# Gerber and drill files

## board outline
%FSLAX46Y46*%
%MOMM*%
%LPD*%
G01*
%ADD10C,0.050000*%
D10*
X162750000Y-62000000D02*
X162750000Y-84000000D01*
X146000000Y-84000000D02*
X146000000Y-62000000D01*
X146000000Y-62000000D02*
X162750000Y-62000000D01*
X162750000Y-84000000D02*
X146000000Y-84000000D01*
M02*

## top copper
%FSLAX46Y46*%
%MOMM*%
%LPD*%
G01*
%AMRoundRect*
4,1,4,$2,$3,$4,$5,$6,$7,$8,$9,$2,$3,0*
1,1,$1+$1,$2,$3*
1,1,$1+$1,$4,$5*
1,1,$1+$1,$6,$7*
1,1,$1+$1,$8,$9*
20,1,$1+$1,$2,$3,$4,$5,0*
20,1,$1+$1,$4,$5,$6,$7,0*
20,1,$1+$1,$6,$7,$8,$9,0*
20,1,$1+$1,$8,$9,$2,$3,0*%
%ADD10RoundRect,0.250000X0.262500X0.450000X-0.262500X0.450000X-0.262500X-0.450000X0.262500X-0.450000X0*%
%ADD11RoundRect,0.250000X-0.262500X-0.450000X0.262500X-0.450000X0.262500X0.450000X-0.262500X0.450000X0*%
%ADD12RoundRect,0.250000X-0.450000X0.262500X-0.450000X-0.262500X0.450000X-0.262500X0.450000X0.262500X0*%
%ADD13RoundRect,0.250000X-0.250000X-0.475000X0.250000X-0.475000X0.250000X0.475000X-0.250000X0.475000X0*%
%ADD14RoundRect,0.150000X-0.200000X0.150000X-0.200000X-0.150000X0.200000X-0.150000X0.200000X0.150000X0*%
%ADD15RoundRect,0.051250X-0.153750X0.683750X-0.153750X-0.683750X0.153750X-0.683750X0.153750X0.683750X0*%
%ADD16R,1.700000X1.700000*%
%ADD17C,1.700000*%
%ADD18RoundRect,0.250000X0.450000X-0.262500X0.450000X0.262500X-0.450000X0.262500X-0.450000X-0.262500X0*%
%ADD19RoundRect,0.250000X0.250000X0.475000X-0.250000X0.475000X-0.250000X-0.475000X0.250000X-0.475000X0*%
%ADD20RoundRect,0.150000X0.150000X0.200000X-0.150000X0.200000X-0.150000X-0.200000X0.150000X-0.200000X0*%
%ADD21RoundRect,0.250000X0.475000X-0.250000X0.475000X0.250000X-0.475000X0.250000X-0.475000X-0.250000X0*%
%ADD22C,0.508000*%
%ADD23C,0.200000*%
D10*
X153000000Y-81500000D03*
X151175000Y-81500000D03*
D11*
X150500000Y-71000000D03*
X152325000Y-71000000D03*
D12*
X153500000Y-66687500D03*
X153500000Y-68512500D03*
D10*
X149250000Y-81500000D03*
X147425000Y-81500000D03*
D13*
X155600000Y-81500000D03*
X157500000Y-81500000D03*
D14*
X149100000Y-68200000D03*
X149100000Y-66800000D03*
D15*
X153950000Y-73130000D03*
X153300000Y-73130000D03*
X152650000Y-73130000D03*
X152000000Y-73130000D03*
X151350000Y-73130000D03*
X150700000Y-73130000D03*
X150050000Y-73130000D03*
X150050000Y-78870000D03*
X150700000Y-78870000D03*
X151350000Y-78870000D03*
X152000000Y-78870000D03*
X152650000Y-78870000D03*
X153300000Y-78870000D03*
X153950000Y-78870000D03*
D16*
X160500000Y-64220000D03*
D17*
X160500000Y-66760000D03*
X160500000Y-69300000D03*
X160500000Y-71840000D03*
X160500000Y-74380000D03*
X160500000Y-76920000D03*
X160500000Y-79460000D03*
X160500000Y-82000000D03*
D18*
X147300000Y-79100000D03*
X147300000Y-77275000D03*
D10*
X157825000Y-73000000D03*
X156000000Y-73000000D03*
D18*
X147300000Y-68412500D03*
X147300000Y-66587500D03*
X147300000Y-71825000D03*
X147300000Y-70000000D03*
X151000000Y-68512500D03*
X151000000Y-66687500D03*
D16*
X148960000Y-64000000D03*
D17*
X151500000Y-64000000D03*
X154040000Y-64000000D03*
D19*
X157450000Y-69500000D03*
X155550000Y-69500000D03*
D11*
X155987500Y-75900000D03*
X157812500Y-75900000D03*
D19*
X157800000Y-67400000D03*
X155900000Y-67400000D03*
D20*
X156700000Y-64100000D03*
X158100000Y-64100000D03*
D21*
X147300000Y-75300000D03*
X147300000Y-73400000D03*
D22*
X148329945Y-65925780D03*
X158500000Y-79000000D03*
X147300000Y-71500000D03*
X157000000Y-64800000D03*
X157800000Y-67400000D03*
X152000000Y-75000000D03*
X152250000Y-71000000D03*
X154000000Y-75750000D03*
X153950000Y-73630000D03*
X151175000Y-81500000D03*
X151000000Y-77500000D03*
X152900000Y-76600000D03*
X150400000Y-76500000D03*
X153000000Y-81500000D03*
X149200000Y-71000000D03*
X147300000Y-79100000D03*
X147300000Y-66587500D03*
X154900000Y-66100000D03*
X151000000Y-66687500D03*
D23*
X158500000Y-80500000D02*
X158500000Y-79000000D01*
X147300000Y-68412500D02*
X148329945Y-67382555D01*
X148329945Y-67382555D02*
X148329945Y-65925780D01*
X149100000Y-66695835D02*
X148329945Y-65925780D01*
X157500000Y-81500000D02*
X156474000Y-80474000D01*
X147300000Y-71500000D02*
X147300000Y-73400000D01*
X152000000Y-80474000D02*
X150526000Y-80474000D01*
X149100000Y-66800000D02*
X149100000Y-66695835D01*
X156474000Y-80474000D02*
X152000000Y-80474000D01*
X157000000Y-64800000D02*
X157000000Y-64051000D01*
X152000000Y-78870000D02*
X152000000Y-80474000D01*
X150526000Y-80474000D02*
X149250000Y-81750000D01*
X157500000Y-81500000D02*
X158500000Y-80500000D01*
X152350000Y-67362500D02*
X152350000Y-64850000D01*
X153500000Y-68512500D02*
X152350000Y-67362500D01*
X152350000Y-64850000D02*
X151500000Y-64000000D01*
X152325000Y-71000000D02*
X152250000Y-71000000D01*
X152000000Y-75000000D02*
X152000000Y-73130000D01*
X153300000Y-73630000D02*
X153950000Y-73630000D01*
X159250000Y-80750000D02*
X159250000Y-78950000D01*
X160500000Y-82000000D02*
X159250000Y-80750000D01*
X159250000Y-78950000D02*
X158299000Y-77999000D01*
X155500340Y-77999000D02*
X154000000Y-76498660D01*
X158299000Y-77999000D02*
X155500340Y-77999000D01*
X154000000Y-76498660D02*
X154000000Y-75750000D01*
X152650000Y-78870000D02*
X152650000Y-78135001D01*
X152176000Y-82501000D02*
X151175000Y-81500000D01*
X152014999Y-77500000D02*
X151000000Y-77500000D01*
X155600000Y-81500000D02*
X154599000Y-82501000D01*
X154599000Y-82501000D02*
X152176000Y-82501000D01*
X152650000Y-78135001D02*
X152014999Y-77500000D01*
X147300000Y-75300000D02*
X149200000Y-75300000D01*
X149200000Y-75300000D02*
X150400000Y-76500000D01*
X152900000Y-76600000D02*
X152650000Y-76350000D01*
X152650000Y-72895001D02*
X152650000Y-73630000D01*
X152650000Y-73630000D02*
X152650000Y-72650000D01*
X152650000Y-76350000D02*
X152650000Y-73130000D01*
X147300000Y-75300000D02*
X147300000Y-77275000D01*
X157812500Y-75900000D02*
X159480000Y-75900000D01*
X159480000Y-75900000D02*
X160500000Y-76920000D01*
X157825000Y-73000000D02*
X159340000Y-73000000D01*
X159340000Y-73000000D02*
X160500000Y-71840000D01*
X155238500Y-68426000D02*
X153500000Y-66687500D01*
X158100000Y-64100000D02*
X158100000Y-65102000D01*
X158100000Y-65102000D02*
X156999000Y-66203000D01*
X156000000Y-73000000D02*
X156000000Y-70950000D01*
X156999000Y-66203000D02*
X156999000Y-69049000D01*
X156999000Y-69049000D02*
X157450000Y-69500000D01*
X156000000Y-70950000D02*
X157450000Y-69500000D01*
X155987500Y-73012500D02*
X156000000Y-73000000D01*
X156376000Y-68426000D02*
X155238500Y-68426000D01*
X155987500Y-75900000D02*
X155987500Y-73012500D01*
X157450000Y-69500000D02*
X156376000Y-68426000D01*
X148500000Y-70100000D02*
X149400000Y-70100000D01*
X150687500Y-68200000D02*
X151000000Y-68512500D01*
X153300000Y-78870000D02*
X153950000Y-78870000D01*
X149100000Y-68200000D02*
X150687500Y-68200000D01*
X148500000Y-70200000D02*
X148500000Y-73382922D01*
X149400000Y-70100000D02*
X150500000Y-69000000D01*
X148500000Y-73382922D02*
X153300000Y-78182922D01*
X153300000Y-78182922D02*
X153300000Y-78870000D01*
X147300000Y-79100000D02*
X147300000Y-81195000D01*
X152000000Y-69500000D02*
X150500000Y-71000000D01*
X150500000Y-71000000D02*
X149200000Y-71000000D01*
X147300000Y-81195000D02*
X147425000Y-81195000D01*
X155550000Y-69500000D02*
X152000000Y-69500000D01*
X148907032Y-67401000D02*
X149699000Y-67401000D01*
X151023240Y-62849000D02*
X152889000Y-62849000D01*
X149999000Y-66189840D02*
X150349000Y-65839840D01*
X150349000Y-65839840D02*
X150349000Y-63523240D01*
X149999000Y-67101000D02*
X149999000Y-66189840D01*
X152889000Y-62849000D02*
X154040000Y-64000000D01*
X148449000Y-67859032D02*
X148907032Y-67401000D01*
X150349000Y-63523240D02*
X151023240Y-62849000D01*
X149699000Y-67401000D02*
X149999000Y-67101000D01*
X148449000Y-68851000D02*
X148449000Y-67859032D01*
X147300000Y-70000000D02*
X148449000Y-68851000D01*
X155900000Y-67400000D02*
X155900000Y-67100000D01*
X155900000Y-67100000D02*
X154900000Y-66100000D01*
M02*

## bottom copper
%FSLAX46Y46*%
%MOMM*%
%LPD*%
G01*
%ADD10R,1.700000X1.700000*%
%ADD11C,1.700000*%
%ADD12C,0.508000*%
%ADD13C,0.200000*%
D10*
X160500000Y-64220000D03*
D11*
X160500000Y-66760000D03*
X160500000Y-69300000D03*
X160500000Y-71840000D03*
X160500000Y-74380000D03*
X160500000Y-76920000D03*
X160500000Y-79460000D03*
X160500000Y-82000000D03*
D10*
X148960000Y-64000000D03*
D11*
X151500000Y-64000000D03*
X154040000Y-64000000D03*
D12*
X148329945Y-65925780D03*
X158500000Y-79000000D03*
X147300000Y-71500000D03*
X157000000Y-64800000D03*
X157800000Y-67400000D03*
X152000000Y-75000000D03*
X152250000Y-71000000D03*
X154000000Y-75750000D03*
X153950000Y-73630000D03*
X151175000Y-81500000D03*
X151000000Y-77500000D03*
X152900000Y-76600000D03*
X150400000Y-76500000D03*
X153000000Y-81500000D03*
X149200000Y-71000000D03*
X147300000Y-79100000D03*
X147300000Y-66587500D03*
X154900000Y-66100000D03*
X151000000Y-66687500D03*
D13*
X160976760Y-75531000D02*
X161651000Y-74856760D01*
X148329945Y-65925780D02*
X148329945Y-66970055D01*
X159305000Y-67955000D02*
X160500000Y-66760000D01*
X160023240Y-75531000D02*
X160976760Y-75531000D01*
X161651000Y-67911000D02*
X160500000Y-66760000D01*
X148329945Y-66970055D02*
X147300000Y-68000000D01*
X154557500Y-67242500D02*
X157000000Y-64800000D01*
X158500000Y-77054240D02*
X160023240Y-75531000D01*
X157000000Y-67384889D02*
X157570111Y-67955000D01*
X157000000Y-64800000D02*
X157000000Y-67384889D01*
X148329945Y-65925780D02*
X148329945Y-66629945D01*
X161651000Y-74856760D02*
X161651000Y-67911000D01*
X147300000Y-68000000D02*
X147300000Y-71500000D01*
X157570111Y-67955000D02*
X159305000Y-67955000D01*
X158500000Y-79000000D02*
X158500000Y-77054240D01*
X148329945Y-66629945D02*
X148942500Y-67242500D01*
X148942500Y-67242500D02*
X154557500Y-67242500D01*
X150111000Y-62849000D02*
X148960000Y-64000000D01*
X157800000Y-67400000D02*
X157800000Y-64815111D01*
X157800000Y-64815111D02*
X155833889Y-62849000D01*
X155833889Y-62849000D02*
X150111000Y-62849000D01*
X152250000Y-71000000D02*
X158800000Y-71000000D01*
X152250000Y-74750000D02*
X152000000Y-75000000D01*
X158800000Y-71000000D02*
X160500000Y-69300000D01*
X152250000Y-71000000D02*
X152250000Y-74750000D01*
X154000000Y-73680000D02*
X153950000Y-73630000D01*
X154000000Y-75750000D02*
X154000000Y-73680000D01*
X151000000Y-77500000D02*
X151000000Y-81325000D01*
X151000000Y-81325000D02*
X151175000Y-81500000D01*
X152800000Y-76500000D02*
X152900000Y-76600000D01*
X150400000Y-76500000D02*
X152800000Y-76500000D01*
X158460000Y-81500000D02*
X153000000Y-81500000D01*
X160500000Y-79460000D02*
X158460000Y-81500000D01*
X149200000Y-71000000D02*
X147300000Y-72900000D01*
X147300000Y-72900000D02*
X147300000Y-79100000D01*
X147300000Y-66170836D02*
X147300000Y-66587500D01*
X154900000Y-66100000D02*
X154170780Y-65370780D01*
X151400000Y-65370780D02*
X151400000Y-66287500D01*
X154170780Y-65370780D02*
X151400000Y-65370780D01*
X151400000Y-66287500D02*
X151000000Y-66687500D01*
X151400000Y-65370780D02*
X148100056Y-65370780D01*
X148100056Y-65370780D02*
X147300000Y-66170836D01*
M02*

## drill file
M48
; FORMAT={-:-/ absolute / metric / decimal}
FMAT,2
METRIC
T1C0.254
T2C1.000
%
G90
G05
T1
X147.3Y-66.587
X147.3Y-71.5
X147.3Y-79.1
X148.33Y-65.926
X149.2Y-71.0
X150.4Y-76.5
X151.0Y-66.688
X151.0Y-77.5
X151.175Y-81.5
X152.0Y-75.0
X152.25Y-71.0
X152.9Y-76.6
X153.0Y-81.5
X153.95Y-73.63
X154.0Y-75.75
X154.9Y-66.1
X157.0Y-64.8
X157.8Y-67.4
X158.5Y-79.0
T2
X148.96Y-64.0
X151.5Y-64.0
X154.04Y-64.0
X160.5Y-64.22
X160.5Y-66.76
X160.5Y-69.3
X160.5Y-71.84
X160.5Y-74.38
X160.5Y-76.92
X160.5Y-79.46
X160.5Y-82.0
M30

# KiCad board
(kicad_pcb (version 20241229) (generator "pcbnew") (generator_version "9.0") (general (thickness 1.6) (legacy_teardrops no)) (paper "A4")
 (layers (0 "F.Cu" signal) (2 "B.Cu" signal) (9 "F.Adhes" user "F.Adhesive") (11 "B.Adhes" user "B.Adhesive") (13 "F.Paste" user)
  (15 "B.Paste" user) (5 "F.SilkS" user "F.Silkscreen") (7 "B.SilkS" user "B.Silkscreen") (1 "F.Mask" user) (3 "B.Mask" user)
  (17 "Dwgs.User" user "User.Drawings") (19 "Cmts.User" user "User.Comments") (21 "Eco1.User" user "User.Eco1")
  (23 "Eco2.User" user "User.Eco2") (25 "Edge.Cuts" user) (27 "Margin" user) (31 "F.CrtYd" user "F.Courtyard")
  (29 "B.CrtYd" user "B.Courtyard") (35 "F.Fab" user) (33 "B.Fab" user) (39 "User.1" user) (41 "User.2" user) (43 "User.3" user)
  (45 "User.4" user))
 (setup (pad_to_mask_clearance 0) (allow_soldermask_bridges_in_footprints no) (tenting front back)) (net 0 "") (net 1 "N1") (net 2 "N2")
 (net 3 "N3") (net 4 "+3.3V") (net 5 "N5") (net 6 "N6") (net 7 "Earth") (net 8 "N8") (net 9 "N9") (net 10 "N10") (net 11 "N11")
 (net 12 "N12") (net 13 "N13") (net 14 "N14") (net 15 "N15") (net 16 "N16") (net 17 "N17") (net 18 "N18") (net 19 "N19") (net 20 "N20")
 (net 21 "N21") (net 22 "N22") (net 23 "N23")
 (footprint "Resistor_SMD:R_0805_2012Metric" (layer "F.Cu") (at 152.0875 81.5 180)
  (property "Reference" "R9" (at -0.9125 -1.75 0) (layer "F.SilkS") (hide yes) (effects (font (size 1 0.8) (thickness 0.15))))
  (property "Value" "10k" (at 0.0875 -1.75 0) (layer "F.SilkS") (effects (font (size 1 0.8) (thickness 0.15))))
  (pad "1" smd roundrect (at -0.9125 0 180) (size 1.025 1.4) (layers "F.Cu" "F.Mask" "F.Paste") (roundrect_rratio 0.243902) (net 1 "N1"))
  (pad "2" smd roundrect (at 0.9125 0 180) (size 1.025 1.4) (layers "F.Cu" "F.Mask" "F.Paste") (roundrect_rratio 0.243902) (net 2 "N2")))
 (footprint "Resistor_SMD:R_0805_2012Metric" (layer "F.Cu") (at 151.4125 71)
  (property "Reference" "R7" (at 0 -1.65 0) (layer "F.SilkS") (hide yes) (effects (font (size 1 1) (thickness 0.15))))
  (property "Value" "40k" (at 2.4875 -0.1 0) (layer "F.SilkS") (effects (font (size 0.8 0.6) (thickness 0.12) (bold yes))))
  (pad "1" smd roundrect (at -0.9125 0) (size 1.025 1.4) (layers "F.Cu" "F.Mask" "F.Paste") (roundrect_rratio 0.243902) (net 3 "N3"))
  (pad "2" smd roundrect (at 0.9125 0) (size 1.025 1.4) (layers "F.Cu" "F.Mask" "F.Paste") (roundrect_rratio 0.243902) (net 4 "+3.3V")))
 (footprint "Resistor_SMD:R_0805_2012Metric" (layer "F.Cu") (at 153.5 67.6 -90)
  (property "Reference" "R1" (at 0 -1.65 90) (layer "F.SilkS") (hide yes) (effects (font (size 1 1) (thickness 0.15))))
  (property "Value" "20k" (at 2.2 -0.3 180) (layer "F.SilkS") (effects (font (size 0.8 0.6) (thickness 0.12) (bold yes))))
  (pad "1" smd roundrect (at -0.9125 0 270) (size 1.025 1.4) (layers "F.Cu" "F.Mask" "F.Paste") (roundrect_rratio 0.243902) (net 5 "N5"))
  (pad "2" smd roundrect (at 0.9125 0 270) (size 1.025 1.4) (layers "F.Cu" "F.Mask" "F.Paste") (roundrect_rratio 0.243902) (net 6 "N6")))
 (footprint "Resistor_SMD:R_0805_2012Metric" (layer "F.Cu") (at 148.3375 81.5 180)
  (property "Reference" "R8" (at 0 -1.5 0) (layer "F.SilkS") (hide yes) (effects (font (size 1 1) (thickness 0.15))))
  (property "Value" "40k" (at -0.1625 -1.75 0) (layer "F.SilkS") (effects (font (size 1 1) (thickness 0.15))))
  (pad "1" smd roundrect (at -0.9125 0 180) (size 1.025 1.4) (layers "F.Cu" "F.Mask" "F.Paste") (roundrect_rratio 0.243902) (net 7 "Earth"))
  (pad "2" smd roundrect (at 0.9125 0 180) (size 1.025 1.4) (layers "F.Cu" "F.Mask" "F.Paste") (roundrect_rratio 0.243902) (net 3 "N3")))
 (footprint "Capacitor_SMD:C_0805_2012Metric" (layer "F.Cu") (at 156.55 81.5)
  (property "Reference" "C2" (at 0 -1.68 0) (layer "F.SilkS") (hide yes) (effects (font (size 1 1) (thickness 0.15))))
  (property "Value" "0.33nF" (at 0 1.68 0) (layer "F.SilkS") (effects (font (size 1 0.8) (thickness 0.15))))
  (pad "1" smd roundrect (at -0.95 0) (size 1 1.45) (layers "F.Cu" "F.Mask" "F.Paste") (roundrect_rratio 0.25) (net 2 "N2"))
  (pad "2" smd roundrect (at 0.95 0) (size 1 1.45) (layers "F.Cu" "F.Mask" "F.Paste") (roundrect_rratio 0.25) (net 7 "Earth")))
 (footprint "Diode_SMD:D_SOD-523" (layer "F.Cu") (at 149.1 67.5 90)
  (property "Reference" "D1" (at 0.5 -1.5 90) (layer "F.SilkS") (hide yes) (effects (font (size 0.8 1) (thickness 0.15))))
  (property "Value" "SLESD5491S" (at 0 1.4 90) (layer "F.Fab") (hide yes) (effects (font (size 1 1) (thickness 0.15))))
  (pad "1" smd roundrect (at -0.7 0 270) (size 0.6 0.7) (layers "F.Cu" "F.Mask" "F.Paste") (roundrect_rratio 0.25) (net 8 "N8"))
  (pad "2" smd roundrect (at 0.7 0 270) (size 0.6 0.7) (layers "F.Cu" "F.Mask" "F.Paste") (roundrect_rratio 0.25) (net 7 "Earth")))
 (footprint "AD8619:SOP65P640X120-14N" (layer "F.Cu") (at 152 76 -90)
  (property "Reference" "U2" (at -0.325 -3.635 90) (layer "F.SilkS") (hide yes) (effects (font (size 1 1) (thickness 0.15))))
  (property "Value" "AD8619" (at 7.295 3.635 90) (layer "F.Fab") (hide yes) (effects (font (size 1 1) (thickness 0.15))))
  (pad "1" smd roundrect (at -2.87 -1.95 270) (size 1.47 0.41) (layers "F.Cu" "F.Mask" "F.Paste") (roundrect_rratio 0.125) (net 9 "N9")
   (solder_mask_margin 0.102))
  (pad "2" smd roundrect (at -2.87 -1.3 270) (size 1.47 0.41) (layers "F.Cu" "F.Mask" "F.Paste") (roundrect_rratio 0.125) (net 9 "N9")
   (solder_mask_margin 0.102))
  (pad "3" smd roundrect (at -2.87 -0.65 270) (size 1.47 0.41) (layers "F.Cu" "F.Mask" "F.Paste") (roundrect_rratio 0.125) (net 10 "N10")
   (solder_mask_margin 0.102))
  (pad "4" smd roundrect (at -2.87 0 270) (size 1.47 0.41) (layers "F.Cu" "F.Mask" "F.Paste") (roundrect_rratio 0.125) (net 4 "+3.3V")
   (solder_mask_margin 0.102))
  (pad "5" smd roundrect (at -2.87 0.65 270) (size 1.47 0.41) (layers "F.Cu" "F.Mask" "F.Paste") (roundrect_rratio 0.125) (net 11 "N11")
   (solder_mask_margin 0.102))
  (pad "6" smd roundrect (at -2.87 1.3 270) (size 1.47 0.41) (layers "F.Cu" "F.Mask" "F.Paste") (roundrect_rratio 0.125) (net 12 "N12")
   (solder_mask_margin 0.102))
  (pad "7" smd roundrect (at -2.87 1.95 270) (size 1.47 0.41) (layers "F.Cu" "F.Mask" "F.Paste") (roundrect_rratio 0.125) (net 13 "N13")
   (solder_mask_margin 0.102))
  (pad "8" smd roundrect (at 2.87 1.95 270) (size 1.47 0.41) (layers "F.Cu" "F.Mask" "F.Paste") (roundrect_rratio 0.125) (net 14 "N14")
   (solder_mask_margin 0.102))
  (pad "9" smd roundrect (at 2.87 1.3 270) (size 1.47 0.41) (layers "F.Cu" "F.Mask" "F.Paste") (roundrect_rratio 0.125) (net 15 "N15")
   (solder_mask_margin 0.102))
  (pad "10" smd roundrect (at 2.87 0.65 270) (size 1.47 0.41) (layers "F.Cu" "F.Mask" "F.Paste") (roundrect_rratio 0.125) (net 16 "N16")
   (solder_mask_margin 0.102))
  (pad "11" smd roundrect (at 2.87 0 270) (size 1.47 0.41) (layers "F.Cu" "F.Mask" "F.Paste") (roundrect_rratio 0.125) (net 7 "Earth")
   (solder_mask_margin 0.102))
  (pad "12" smd roundrect (at 2.87 -0.65 270) (size 1.47 0.41) (layers "F.Cu" "F.Mask" "F.Paste") (roundrect_rratio 0.125) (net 2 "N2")
   (solder_mask_margin 0.102))
  (pad "13" smd roundrect (at 2.87 -1.3 270) (size 1.47 0.41) (layers "F.Cu" "F.Mask" "F.Paste") (roundrect_rratio 0.125) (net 8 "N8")
   (solder_mask_margin 0.102))
  (pad "14" smd roundrect (at 2.87 -1.95 270) (size 1.47 0.41) (layers "F.Cu" "F.Mask" "F.Paste") (roundrect_rratio 0.125) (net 8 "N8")
   (solder_mask_margin 0.102)))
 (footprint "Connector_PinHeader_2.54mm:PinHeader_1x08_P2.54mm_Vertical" (layer "F.Cu") (at 160.5 64.22)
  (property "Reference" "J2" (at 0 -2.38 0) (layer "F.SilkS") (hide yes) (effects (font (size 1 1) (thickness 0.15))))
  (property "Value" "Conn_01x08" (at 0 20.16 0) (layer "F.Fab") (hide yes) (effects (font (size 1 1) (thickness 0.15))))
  (pad "1" thru_hole rect (at 0 0) (size 1.7 1.7) (drill 1) (layers "*.Cu" "*.Mask") (remove_unused_layers no) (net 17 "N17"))
  (pad "2" thru_hole circle (at 0 2.54) (size 1.7 1.7) (drill 1) (layers "*.Cu" "*.Mask") (remove_unused_layers no) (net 7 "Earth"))
  (pad "3" thru_hole circle (at 0 5.08) (size 1.7 1.7) (drill 1) (layers "*.Cu" "*.Mask") (remove_unused_layers no) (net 4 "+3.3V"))
  (pad "4" thru_hole circle (at 0 7.62) (size 1.7 1.7) (drill 1) (layers "*.Cu" "*.Mask") (remove_unused_layers no) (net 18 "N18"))
  (pad "5" thru_hole circle (at 0 10.16) (size 1.7 1.7) (drill 1) (layers "*.Cu" "*.Mask") (remove_unused_layers no) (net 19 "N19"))
  (pad "6" thru_hole circle (at 0 12.7) (size 1.7 1.7) (drill 1) (layers "*.Cu" "*.Mask") (remove_unused_layers no) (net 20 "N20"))
  (pad "7" thru_hole circle (at 0 15.24) (size 1.7 1.7) (drill 1) (layers "*.Cu" "*.Mask") (remove_unused_layers no) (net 1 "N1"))
  (pad "8" thru_hole circle (at 0 17.78) (size 1.7 1.7) (drill 1) (layers "*.Cu" "*.Mask") (remove_unused_layers no) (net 9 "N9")))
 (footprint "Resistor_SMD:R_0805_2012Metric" (layer "F.Cu") (at 147.3 78.1875 90)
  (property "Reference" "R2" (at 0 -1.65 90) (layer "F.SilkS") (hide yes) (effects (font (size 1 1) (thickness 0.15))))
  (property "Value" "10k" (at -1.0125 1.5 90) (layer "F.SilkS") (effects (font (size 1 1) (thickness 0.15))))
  (pad "1" smd roundrect (at -0.9125 0 90) (size 1.025 1.4) (layers "F.Cu" "F.Mask" "F.Paste") (roundrect_rratio 0.243902) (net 3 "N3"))
  (pad "2" smd roundrect (at 0.9125 0 90) (size 1.025 1.4) (layers "F.Cu" "F.Mask" "F.Paste") (roundrect_rratio 0.243902) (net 10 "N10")))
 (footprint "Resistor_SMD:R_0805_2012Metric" (layer "F.Cu") (at 156.9125 73 180)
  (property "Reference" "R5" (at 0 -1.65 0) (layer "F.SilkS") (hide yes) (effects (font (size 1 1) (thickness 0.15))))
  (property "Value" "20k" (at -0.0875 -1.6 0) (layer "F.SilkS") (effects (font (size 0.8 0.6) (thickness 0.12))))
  (pad "1" smd roundrect (at -0.9125 0 180) (size 1.025 1.4) (layers "F.Cu" "F.Mask" "F.Paste") (roundrect_rratio 0.243902) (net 18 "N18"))
  (pad "2" smd roundrect (at 0.9125 0 180) (size 1.025 1.4) (layers "F.Cu" "F.Mask" "F.Paste") (roundrect_rratio 0.243902) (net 5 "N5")))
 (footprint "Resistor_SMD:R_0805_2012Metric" (layer "F.Cu") (at 147.3 67.5 90)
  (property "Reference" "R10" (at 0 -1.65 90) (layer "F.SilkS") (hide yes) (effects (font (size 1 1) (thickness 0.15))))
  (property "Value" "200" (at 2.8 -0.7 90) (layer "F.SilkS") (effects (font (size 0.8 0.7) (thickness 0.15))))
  (pad "1" smd roundrect (at -0.9125 0 90) (size 1.025 1.4) (layers "F.Cu" "F.Mask" "F.Paste") (roundrect_rratio 0.243902) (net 7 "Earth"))
  (pad "2" smd roundrect (at 0.9125 0 90) (size 1.025 1.4) (layers "F.Cu" "F.Mask" "F.Paste") (roundrect_rratio 0.243902) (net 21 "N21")))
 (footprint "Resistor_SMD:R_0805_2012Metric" (layer "F.Cu") (at 147.3 70.9125 90)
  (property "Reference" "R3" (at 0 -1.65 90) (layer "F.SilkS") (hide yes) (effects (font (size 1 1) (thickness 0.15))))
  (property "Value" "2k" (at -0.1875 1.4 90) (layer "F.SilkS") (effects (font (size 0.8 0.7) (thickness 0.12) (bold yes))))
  (pad "1" smd roundrect (at -0.9125 0 90) (size 1.025 1.4) (layers "F.Cu" "F.Mask" "F.Paste") (roundrect_rratio 0.243902) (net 7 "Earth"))
  (pad "2" smd roundrect (at 0.9125 0 90) (size 1.025 1.4) (layers "F.Cu" "F.Mask" "F.Paste") (roundrect_rratio 0.243902) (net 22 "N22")))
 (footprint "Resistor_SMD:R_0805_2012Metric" (layer "F.Cu") (at 151 67.6 90)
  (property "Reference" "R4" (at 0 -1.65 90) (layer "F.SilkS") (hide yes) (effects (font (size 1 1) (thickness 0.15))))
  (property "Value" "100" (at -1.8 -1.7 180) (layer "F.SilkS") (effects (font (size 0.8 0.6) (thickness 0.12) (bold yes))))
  (pad "1" smd roundrect (at -0.9125 0 90) (size 1.025 1.4) (layers "F.Cu" "F.Mask" "F.Paste") (roundrect_rratio 0.243902) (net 8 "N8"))
  (pad "2" smd roundrect (at 0.9125 0 90) (size 1.025 1.4) (layers "F.Cu" "F.Mask" "F.Paste") (roundrect_rratio 0.243902) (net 21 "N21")))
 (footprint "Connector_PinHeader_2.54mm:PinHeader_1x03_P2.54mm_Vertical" (layer "F.Cu") (at 148.96 64 90)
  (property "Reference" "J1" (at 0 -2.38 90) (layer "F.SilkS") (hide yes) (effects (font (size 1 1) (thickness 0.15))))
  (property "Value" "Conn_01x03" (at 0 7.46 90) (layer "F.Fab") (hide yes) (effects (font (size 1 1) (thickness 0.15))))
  (pad "1" thru_hole rect (at 0 0 90) (size 1.7 1.7) (drill 1) (layers "*.Cu" "*.Mask") (remove_unused_layers no) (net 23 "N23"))
  (pad "2" thru_hole circle (at 0 2.54 90) (size 1.7 1.7) (drill 1) (layers "*.Cu" "*.Mask") (remove_unused_layers no) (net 6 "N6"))
  (pad "3" thru_hole circle (at 0 5.08 90) (size 1.7 1.7) (drill 1) (layers "*.Cu" "*.Mask") (remove_unused_layers no) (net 22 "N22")))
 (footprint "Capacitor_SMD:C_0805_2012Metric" (layer "F.Cu") (at 156.5 69.5 180)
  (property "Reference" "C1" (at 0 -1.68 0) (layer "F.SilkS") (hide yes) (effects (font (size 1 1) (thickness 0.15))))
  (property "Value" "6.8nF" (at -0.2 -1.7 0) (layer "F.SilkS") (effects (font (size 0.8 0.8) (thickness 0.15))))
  (pad "1" smd roundrect (at -0.95 0 180) (size 1 1.45) (layers "F.Cu" "F.Mask" "F.Paste") (roundrect_rratio 0.25) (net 5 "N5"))
  (pad "2" smd roundrect (at 0.95 0 180) (size 1 1.45) (layers "F.Cu" "F.Mask" "F.Paste") (roundrect_rratio 0.25) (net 3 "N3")))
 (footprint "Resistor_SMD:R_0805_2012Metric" (layer "F.Cu") (at 156.9 75.9)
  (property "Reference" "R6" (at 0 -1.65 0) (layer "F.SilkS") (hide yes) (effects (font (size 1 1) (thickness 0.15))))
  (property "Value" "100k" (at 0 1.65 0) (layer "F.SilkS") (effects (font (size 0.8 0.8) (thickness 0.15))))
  (pad "1" smd roundrect (at -0.9125 0) (size 1.025 1.4) (layers "F.Cu" "F.Mask" "F.Paste") (roundrect_rratio 0.243902) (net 5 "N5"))
  (pad "2" smd roundrect (at 0.9125 0) (size 1.025 1.4) (layers "F.Cu" "F.Mask" "F.Paste") (roundrect_rratio 0.243902) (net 20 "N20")))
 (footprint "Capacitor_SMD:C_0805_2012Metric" (layer "F.Cu") (at 156.85 67.4 180)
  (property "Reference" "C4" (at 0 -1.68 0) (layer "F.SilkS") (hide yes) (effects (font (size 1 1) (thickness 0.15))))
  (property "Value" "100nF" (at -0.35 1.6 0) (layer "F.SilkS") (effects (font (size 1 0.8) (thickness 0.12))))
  (pad "1" smd roundrect (at -0.95 0 180) (size 1 1.45) (layers "F.Cu" "F.Mask" "F.Paste") (roundrect_rratio 0.25) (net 23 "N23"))
  (pad "2" smd roundrect (at 0.95 0 180) (size 1 1.45) (layers "F.Cu" "F.Mask" "F.Paste") (roundrect_rratio 0.25) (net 21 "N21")))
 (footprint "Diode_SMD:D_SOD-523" (layer "F.Cu") (at 157.4 64.1)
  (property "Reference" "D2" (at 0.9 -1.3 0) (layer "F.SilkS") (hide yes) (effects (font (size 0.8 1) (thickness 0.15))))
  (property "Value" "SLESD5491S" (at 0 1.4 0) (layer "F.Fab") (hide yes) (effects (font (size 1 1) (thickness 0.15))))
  (pad "1" smd roundrect (at -0.7 0 180) (size 0.6 0.7) (layers "F.Cu" "F.Mask" "F.Paste") (roundrect_rratio 0.25) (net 7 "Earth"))
  (pad "2" smd roundrect (at 0.7 0 180) (size 0.6 0.7) (layers "F.Cu" "F.Mask" "F.Paste") (roundrect_rratio 0.25) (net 5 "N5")))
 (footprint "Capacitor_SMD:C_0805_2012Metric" (layer "F.Cu") (at 147.3 74.35 90)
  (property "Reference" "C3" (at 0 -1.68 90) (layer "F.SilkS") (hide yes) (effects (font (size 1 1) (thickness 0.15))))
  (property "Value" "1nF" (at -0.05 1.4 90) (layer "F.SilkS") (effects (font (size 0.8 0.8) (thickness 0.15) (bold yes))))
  (pad "1" smd roundrect (at -0.95 0 90) (size 1 1.45) (layers "F.Cu" "F.Mask" "F.Paste") (roundrect_rratio 0.25) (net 10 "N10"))
  (pad "2" smd roundrect (at 0.95 0 90) (size 1 1.45) (layers "F.Cu" "F.Mask" "F.Paste") (roundrect_rratio 0.25) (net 7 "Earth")))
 (gr_line (start 162.75 62) (end 162.75 84) (stroke (width 0.05) (type default)) (layer "Edge.Cuts"))
 (gr_line (start 146 84) (end 146 62) (stroke (width 0.05) (type default)) (layer "Edge.Cuts"))
 (gr_line (start 146 62) (end 162.75 62) (stroke (width 0.05) (type default)) (layer "Edge.Cuts"))
 (gr_line (start 162.75 84) (end 146 84) (stroke (width 0.05) (type default)) (layer "Edge.Cuts"))
 (segment (start 158.5 80.5) (end 158.5 79) (width 0.2) (layer "F.Cu") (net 7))
 (segment (start 147.3 68.4125) (end 148.329945 67.382555) (width 0.2) (layer "F.Cu") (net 7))
 (segment (start 148.329945 67.382555) (end 148.329945 65.92578) (width 0.2) (layer "F.Cu") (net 7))
 (segment (start 149.1 66.695835) (end 148.329945 65.92578) (width 0.2) (layer "F.Cu") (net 7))
 (segment (start 157.5 81.5) (end 156.474 80.474) (width 0.2) (layer "F.Cu") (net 7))
 (segment (start 147.3 71.5) (end 147.3 73.4) (width 0.2) (layer "F.Cu") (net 7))
 (segment (start 152 80.474) (end 150.526 80.474) (width 0.2) (layer "F.Cu") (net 7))
 (segment (start 149.1 66.8) (end 149.1 66.695835) (width 0.2) (layer "F.Cu") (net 7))
 (segment (start 156.474 80.474) (end 152 80.474) (width 0.2) (layer "F.Cu") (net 7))
 (segment (start 157 64.8) (end 157 64.051) (width 0.2) (layer "F.Cu") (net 7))
 (segment (start 152 78.87) (end 152 80.474) (width 0.2) (layer "F.Cu") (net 7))
 (segment (start 150.526 80.474) (end 149.25 81.75) (width 0.2) (layer "F.Cu") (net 7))
 (segment (start 157.5 81.5) (end 158.5 80.5) (width 0.2) (layer "F.Cu") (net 7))
 (via micro (at 148.329945 65.92578) (size 0.508) (drill 0.254) (layers "F.Cu" "B.Cu") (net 7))
 (via micro (at 158.5 79) (size 0.508) (drill 0.254) (layers "F.Cu" "B.Cu") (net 7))
 (via micro (at 147.3 71.5) (size 0.508) (drill 0.254) (layers "F.Cu" "B.Cu") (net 7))
 (via micro (at 157 64.8) (size 0.508) (drill 0.254) (layers "F.Cu" "B.Cu") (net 7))
 (segment (start 160.97676 75.531) (end 161.651 74.85676) (width 0.2) (layer "B.Cu") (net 7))
 (segment (start 148.329945 65.92578) (end 148.329945 66.970055) (width 0.2) (layer "B.Cu") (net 7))
 (segment (start 159.305 67.955) (end 160.5 66.76) (width 0.2) (layer "B.Cu") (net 7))
 (segment (start 160.02324 75.531) (end 160.97676 75.531) (width 0.2) (layer "B.Cu") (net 7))
 (segment (start 161.651 67.911) (end 160.5 66.76) (width 0.2) (layer "B.Cu") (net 7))
 (segment (start 148.329945 66.970055) (end 147.3 68) (width 0.2) (layer "B.Cu") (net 7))
 (segment (start 154.5575 67.2425) (end 157 64.8) (width 0.2) (layer "B.Cu") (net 7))
 (segment (start 158.5 77.05424) (end 160.02324 75.531) (width 0.2) (layer "B.Cu") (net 7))
 (segment (start 157 67.384889) (end 157.570111 67.955) (width 0.2) (layer "B.Cu") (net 7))
 (segment (start 157 64.8) (end 157 67.384889) (width 0.2) (layer "B.Cu") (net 7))
 (segment (start 148.329945 65.92578) (end 148.329945 66.629945) (width 0.2) (layer "B.Cu") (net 7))
 (segment (start 161.651 74.85676) (end 161.651 67.911) (width 0.2) (layer "B.Cu") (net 7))
 (segment (start 147.3 68) (end 147.3 71.5) (width 0.2) (layer "B.Cu") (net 7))
 (segment (start 157.570111 67.955) (end 159.305 67.955) (width 0.2) (layer "B.Cu") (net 7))
 (segment (start 158.5 79) (end 158.5 77.05424) (width 0.2) (layer "B.Cu") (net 7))
 (segment (start 148.329945 66.629945) (end 148.9425 67.2425) (width 0.2) (layer "B.Cu") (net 7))
 (segment (start 148.9425 67.2425) (end 154.5575 67.2425) (width 0.2) (layer "B.Cu") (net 7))
 (segment (start 152.35 67.3625) (end 152.35 64.85) (width 0.2) (layer "F.Cu") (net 6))
 (segment (start 153.5 68.5125) (end 152.35 67.3625) (width 0.2) (layer "F.Cu") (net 6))
 (segment (start 152.35 64.85) (end 151.5 64) (width 0.2) (layer "F.Cu") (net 6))
 (via micro (at 157.8 67.4) (size 0.508) (drill 0.254) (layers "F.Cu" "B.Cu") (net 23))
 (segment (start 150.111 62.849) (end 148.96 64) (width 0.2) (layer "B.Cu") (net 23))
 (segment (start 157.8 67.4) (end 157.8 64.815111) (width 0.2) (layer "B.Cu") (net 23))
 (segment (start 157.8 64.815111) (end 155.833889 62.849) (width 0.2) (layer "B.Cu") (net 23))
 (segment (start 155.833889 62.849) (end 150.111 62.849) (width 0.2) (layer "B.Cu") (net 23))
 (segment (start 152.325 71) (end 152.25 71) (width 0.2) (layer "F.Cu") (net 4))
 (segment (start 152 75) (end 152 73.13) (width 0.2) (layer "F.Cu") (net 4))
 (via micro (at 152 75) (size 0.508) (drill 0.254) (layers "F.Cu" "B.Cu") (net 4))
 (via micro (at 152.25 71) (size 0.508) (drill 0.254) (layers "F.Cu" "B.Cu") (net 4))
 (segment (start 152.25 71) (end 158.8 71) (width 0.2) (layer "B.Cu") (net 4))
 (segment (start 152.25 74.75) (end 152 75) (width 0.2) (layer "B.Cu") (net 4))
 (segment (start 158.8 71) (end 160.5 69.3) (width 0.2) (layer "B.Cu") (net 4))
 (segment (start 152.25 71) (end 152.25 74.75) (width 0.2) (layer "B.Cu") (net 4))
 (segment (start 153.3 73.63) (end 153.95 73.63) (width 0.2) (layer "F.Cu") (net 9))
 (segment (start 159.25 80.75) (end 159.25 78.95) (width 0.2) (layer "F.Cu") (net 9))
 (segment (start 160.5 82) (end 159.25 80.75) (width 0.2) (layer "F.Cu") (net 9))
 (segment (start 159.25 78.95) (end 158.299 77.999) (width 0.2) (layer "F.Cu") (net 9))
 (segment (start 155.50034 77.999) (end 154 76.49866) (width 0.2) (layer "F.Cu") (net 9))
 (segment (start 158.299 77.999) (end 155.50034 77.999) (width 0.2) (layer "F.Cu") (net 9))
 (segment (start 154 76.49866) (end 154 75.75) (width 0.2) (layer "F.Cu") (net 9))
 (via micro (at 154 75.75) (size 0.508) (drill 0.254) (layers "F.Cu" "B.Cu") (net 9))
 (via micro (at 153.95 73.63) (size 0.508) (drill 0.254) (layers "F.Cu" "B.Cu") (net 9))
 (segment (start 154 73.68) (end 153.95 73.63) (width 0.2) (layer "B.Cu") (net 9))
 (segment (start 154 75.75) (end 154 73.68) (width 0.2) (layer "B.Cu") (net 9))
 (segment (start 152.65 78.87) (end 152.65 78.135001) (width 0.2) (layer "F.Cu") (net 2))
 (segment (start 152.176 82.501) (end 151.175 81.5) (width 0.2) (layer "F.Cu") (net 2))
 (segment (start 152.014999 77.5) (end 151 77.5) (width 0.2) (layer "F.Cu") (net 2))
 (segment (start 155.6 81.5) (end 154.599 82.501) (width 0.2) (layer "F.Cu") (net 2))
 (segment (start 154.599 82.501) (end 152.176 82.501) (width 0.2) (layer "F.Cu") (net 2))
 (segment (start 152.65 78.135001) (end 152.014999 77.5) (width 0.2) (layer "F.Cu") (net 2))
 (via micro (at 151.175 81.5) (size 0.508) (drill 0.254) (layers "F.Cu" "B.Cu") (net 2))
 (via micro (at 151 77.5) (size 0.508) (drill 0.254) (layers "F.Cu" "B.Cu") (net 2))
 (segment (start 151 77.5) (end 151 81.325) (width 0.2) (layer "B.Cu") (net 2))
 (segment (start 151 81.325) (end 151.175 81.5) (width 0.2) (layer "B.Cu") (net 2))
 (segment (start 147.3 75.3) (end 149.2 75.3) (width 0.2) (layer "F.Cu") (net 10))
 (segment (start 149.2 75.3) (end 150.4 76.5) (width 0.2) (layer "F.Cu") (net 10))
 (segment (start 152.9 76.6) (end 152.65 76.35) (width 0.2) (layer "F.Cu") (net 10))
 (segment (start 152.65 72.895001) (end 152.65 73.63) (width 0.2) (layer "F.Cu") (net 10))
 (segment (start 152.65 73.63) (end 152.65 72.65) (width 0.2) (layer "F.Cu") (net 10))
 (segment (start 152.65 76.35) (end 152.65 73.13) (width 0.2) (layer "F.Cu") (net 10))
 (segment (start 147.3 75.3) (end 147.3 77.275) (width 0.2) (layer "F.Cu") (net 10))
 (via micro (at 152.9 76.6) (size 0.508) (drill 0.254) (layers "F.Cu" "B.Cu") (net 10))
 (via micro (at 150.4 76.5) (size 0.508) (drill 0.254) (layers "F.Cu" "B.Cu") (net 10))
 (segment (start 152.8 76.5) (end 152.9 76.6) (width 0.2) (layer "B.Cu") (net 10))
 (segment (start 150.4 76.5) (end 152.8 76.5) (width 0.2) (layer "B.Cu") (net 10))
 (via micro (at 153 81.5) (size 0.508) (drill 0.254) (layers "F.Cu" "B.Cu") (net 1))
 (segment (start 158.46 81.5) (end 153 81.5) (width 0.2) (layer "B.Cu") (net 1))
 (segment (start 160.5 79.46) (end 158.46 81.5) (width 0.2) (layer "B.Cu") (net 1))
 (segment (start 157.8125 75.9) (end 159.48 75.9) (width 0.2) (layer "F.Cu") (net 20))
 (segment (start 159.48 75.9) (end 160.5 76.92) (width 0.2) (layer "F.Cu") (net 20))
 (segment (start 157.825 73) (end 159.34 73) (width 0.2) (layer "F.Cu") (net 18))
 (segment (start 159.34 73) (end 160.5 71.84) (width 0.2) (layer "F.Cu") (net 18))
 (segment (start 155.2385 68.426) (end 153.5 66.6875) (width 0.2) (layer "F.Cu") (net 5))
 (segment (start 158.1 64.1) (end 158.1 65.102) (width 0.2) (layer "F.Cu") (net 5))
 (segment (start 158.1 65.102) (end 156.999 66.203) (width 0.2) (layer "F.Cu") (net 5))
 (segment (start 156 73) (end 156 70.95) (width 0.2) (layer "F.Cu") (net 5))
 (segment (start 156.999 66.203) (end 156.999 69.049) (width 0.2) (layer "F.Cu") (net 5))
 (segment (start 156.999 69.049) (end 157.45 69.5) (width 0.2) (layer "F.Cu") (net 5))
 (segment (start 156 70.95) (end 157.45 69.5) (width 0.2) (layer "F.Cu") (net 5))
 (segment (start 155.9875 73.0125) (end 156 73) (width 0.2) (layer "F.Cu") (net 5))
 (segment (start 156.376 68.426) (end 155.2385 68.426) (width 0.2) (layer "F.Cu") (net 5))
 (segment (start 155.9875 75.9) (end 155.9875 73.0125) (width 0.2) (layer "F.Cu") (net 5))
 (segment (start 157.45 69.5) (end 156.376 68.426) (width 0.2) (layer "F.Cu") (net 5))
 (segment (start 148.5 70.1) (end 149.4 70.1) (width 0.2) (layer "F.Cu") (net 8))
 (segment (start 150.6875 68.2) (end 151 68.5125) (width 0.2) (layer "F.Cu") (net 8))
 (segment (start 153.3 78.87) (end 153.95 78.87) (width 0.2) (layer "F.Cu") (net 8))
 (segment (start 149.1 68.2) (end 150.6875 68.2) (width 0.2) (layer "F.Cu") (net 8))
 (segment (start 148.5 70.2) (end 148.5 73.382922) (width 0.2) (layer "F.Cu") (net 8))
 (segment (start 149.4 70.1) (end 150.5 69) (width 0.2) (layer "F.Cu") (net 8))
 (segment (start 148.5 73.382922) (end 153.3 78.182922) (width 0.2) (layer "F.Cu") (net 8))
 (segment (start 153.3 78.182922) (end 153.3 78.87) (width 0.2) (layer "F.Cu") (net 8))
 (segment (start 147.3 79.1) (end 147.3 81.195) (width 0.2) (layer "F.Cu") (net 3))
 (segment (start 152 69.5) (end 150.5 71) (width 0.2) (layer "F.Cu") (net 3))
 (segment (start 150.5 71) (end 149.2 71) (width 0.2) (layer "F.Cu") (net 3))
 (segment (start 147.3 81.195) (end 147.425 81.195) (width 0.2) (layer "F.Cu") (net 3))
 (segment (start 155.55 69.5) (end 152 69.5) (width 0.2) (layer "F.Cu") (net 3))
 (via micro (at 149.2 71) (size 0.508) (drill 0.254) (layers "F.Cu" "B.Cu") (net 3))
 (via micro (at 147.3 79.1) (size 0.508) (drill 0.254) (layers "F.Cu" "B.Cu") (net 3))
 (segment (start 149.2 71) (end 147.3 72.9) (width 0.2) (layer "B.Cu") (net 3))
 (segment (start 147.3 72.9) (end 147.3 79.1) (width 0.2) (layer "B.Cu") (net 3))
 (segment (start 148.907032 67.401) (end 149.699 67.401) (width 0.2) (layer "F.Cu") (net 22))
 (segment (start 151.02324 62.849) (end 152.889 62.849) (width 0.2) (layer "F.Cu") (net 22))
 (segment (start 149.999 66.18984) (end 150.349 65.83984) (width 0.2) (layer "F.Cu") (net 22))
 (segment (start 150.349 65.83984) (end 150.349 63.52324) (width 0.2) (layer "F.Cu") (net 22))
 (segment (start 149.999 67.101) (end 149.999 66.18984) (width 0.2) (layer "F.Cu") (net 22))
 (segment (start 152.889 62.849) (end 154.04 64) (width 0.2) (layer "F.Cu") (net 22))
 (segment (start 148.449 67.859032) (end 148.907032 67.401) (width 0.2) (layer "F.Cu") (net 22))
 (segment (start 150.349 63.52324) (end 151.02324 62.849) (width 0.2) (layer "F.Cu") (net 22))
 (segment (start 149.699 67.401) (end 149.999 67.101) (width 0.2) (layer "F.Cu") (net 22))
 (segment (start 148.449 68.851) (end 148.449 67.859032) (width 0.2) (layer "F.Cu") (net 22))
 (segment (start 147.3 70) (end 148.449 68.851) (width 0.2) (layer "F.Cu") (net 22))
 (segment (start 155.9 67.4) (end 155.9 67.1) (width 0.2) (layer "F.Cu") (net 21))
 (segment (start 155.9 67.1) (end 154.9 66.1) (width 0.2) (layer "F.Cu") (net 21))
 (via micro (at 147.3 66.5875) (size 0.508) (drill 0.254) (layers "F.Cu" "B.Cu") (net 21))
 (via micro (at 154.9 66.1) (size 0.508) (drill 0.254) (layers "F.Cu" "B.Cu") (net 21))
 (via micro (at 151 66.6875) (size 0.508) (drill 0.254) (layers "F.Cu" "B.Cu") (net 21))
 (segment (start 147.3 66.170836) (end 147.3 66.5875) (width 0.2) (layer "B.Cu") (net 21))
 (segment (start 154.9 66.1) (end 154.17078 65.37078) (width 0.2) (layer "B.Cu") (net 21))
 (segment (start 151.4 65.37078) (end 151.4 66.2875) (width 0.2) (layer "B.Cu") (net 21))
 (segment (start 154.17078 65.37078) (end 151.4 65.37078) (width 0.2) (layer "B.Cu") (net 21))
 (segment (start 151.4 66.2875) (end 151 66.6875) (width 0.2) (layer "B.Cu") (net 21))
 (segment (start 151.4 65.37078) (end 148.100056 65.37078) (width 0.2) (layer "B.Cu") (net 21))
 (segment (start 148.100056 65.37078) (end 147.3 66.170836) (width 0.2) (layer "B.Cu") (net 21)))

